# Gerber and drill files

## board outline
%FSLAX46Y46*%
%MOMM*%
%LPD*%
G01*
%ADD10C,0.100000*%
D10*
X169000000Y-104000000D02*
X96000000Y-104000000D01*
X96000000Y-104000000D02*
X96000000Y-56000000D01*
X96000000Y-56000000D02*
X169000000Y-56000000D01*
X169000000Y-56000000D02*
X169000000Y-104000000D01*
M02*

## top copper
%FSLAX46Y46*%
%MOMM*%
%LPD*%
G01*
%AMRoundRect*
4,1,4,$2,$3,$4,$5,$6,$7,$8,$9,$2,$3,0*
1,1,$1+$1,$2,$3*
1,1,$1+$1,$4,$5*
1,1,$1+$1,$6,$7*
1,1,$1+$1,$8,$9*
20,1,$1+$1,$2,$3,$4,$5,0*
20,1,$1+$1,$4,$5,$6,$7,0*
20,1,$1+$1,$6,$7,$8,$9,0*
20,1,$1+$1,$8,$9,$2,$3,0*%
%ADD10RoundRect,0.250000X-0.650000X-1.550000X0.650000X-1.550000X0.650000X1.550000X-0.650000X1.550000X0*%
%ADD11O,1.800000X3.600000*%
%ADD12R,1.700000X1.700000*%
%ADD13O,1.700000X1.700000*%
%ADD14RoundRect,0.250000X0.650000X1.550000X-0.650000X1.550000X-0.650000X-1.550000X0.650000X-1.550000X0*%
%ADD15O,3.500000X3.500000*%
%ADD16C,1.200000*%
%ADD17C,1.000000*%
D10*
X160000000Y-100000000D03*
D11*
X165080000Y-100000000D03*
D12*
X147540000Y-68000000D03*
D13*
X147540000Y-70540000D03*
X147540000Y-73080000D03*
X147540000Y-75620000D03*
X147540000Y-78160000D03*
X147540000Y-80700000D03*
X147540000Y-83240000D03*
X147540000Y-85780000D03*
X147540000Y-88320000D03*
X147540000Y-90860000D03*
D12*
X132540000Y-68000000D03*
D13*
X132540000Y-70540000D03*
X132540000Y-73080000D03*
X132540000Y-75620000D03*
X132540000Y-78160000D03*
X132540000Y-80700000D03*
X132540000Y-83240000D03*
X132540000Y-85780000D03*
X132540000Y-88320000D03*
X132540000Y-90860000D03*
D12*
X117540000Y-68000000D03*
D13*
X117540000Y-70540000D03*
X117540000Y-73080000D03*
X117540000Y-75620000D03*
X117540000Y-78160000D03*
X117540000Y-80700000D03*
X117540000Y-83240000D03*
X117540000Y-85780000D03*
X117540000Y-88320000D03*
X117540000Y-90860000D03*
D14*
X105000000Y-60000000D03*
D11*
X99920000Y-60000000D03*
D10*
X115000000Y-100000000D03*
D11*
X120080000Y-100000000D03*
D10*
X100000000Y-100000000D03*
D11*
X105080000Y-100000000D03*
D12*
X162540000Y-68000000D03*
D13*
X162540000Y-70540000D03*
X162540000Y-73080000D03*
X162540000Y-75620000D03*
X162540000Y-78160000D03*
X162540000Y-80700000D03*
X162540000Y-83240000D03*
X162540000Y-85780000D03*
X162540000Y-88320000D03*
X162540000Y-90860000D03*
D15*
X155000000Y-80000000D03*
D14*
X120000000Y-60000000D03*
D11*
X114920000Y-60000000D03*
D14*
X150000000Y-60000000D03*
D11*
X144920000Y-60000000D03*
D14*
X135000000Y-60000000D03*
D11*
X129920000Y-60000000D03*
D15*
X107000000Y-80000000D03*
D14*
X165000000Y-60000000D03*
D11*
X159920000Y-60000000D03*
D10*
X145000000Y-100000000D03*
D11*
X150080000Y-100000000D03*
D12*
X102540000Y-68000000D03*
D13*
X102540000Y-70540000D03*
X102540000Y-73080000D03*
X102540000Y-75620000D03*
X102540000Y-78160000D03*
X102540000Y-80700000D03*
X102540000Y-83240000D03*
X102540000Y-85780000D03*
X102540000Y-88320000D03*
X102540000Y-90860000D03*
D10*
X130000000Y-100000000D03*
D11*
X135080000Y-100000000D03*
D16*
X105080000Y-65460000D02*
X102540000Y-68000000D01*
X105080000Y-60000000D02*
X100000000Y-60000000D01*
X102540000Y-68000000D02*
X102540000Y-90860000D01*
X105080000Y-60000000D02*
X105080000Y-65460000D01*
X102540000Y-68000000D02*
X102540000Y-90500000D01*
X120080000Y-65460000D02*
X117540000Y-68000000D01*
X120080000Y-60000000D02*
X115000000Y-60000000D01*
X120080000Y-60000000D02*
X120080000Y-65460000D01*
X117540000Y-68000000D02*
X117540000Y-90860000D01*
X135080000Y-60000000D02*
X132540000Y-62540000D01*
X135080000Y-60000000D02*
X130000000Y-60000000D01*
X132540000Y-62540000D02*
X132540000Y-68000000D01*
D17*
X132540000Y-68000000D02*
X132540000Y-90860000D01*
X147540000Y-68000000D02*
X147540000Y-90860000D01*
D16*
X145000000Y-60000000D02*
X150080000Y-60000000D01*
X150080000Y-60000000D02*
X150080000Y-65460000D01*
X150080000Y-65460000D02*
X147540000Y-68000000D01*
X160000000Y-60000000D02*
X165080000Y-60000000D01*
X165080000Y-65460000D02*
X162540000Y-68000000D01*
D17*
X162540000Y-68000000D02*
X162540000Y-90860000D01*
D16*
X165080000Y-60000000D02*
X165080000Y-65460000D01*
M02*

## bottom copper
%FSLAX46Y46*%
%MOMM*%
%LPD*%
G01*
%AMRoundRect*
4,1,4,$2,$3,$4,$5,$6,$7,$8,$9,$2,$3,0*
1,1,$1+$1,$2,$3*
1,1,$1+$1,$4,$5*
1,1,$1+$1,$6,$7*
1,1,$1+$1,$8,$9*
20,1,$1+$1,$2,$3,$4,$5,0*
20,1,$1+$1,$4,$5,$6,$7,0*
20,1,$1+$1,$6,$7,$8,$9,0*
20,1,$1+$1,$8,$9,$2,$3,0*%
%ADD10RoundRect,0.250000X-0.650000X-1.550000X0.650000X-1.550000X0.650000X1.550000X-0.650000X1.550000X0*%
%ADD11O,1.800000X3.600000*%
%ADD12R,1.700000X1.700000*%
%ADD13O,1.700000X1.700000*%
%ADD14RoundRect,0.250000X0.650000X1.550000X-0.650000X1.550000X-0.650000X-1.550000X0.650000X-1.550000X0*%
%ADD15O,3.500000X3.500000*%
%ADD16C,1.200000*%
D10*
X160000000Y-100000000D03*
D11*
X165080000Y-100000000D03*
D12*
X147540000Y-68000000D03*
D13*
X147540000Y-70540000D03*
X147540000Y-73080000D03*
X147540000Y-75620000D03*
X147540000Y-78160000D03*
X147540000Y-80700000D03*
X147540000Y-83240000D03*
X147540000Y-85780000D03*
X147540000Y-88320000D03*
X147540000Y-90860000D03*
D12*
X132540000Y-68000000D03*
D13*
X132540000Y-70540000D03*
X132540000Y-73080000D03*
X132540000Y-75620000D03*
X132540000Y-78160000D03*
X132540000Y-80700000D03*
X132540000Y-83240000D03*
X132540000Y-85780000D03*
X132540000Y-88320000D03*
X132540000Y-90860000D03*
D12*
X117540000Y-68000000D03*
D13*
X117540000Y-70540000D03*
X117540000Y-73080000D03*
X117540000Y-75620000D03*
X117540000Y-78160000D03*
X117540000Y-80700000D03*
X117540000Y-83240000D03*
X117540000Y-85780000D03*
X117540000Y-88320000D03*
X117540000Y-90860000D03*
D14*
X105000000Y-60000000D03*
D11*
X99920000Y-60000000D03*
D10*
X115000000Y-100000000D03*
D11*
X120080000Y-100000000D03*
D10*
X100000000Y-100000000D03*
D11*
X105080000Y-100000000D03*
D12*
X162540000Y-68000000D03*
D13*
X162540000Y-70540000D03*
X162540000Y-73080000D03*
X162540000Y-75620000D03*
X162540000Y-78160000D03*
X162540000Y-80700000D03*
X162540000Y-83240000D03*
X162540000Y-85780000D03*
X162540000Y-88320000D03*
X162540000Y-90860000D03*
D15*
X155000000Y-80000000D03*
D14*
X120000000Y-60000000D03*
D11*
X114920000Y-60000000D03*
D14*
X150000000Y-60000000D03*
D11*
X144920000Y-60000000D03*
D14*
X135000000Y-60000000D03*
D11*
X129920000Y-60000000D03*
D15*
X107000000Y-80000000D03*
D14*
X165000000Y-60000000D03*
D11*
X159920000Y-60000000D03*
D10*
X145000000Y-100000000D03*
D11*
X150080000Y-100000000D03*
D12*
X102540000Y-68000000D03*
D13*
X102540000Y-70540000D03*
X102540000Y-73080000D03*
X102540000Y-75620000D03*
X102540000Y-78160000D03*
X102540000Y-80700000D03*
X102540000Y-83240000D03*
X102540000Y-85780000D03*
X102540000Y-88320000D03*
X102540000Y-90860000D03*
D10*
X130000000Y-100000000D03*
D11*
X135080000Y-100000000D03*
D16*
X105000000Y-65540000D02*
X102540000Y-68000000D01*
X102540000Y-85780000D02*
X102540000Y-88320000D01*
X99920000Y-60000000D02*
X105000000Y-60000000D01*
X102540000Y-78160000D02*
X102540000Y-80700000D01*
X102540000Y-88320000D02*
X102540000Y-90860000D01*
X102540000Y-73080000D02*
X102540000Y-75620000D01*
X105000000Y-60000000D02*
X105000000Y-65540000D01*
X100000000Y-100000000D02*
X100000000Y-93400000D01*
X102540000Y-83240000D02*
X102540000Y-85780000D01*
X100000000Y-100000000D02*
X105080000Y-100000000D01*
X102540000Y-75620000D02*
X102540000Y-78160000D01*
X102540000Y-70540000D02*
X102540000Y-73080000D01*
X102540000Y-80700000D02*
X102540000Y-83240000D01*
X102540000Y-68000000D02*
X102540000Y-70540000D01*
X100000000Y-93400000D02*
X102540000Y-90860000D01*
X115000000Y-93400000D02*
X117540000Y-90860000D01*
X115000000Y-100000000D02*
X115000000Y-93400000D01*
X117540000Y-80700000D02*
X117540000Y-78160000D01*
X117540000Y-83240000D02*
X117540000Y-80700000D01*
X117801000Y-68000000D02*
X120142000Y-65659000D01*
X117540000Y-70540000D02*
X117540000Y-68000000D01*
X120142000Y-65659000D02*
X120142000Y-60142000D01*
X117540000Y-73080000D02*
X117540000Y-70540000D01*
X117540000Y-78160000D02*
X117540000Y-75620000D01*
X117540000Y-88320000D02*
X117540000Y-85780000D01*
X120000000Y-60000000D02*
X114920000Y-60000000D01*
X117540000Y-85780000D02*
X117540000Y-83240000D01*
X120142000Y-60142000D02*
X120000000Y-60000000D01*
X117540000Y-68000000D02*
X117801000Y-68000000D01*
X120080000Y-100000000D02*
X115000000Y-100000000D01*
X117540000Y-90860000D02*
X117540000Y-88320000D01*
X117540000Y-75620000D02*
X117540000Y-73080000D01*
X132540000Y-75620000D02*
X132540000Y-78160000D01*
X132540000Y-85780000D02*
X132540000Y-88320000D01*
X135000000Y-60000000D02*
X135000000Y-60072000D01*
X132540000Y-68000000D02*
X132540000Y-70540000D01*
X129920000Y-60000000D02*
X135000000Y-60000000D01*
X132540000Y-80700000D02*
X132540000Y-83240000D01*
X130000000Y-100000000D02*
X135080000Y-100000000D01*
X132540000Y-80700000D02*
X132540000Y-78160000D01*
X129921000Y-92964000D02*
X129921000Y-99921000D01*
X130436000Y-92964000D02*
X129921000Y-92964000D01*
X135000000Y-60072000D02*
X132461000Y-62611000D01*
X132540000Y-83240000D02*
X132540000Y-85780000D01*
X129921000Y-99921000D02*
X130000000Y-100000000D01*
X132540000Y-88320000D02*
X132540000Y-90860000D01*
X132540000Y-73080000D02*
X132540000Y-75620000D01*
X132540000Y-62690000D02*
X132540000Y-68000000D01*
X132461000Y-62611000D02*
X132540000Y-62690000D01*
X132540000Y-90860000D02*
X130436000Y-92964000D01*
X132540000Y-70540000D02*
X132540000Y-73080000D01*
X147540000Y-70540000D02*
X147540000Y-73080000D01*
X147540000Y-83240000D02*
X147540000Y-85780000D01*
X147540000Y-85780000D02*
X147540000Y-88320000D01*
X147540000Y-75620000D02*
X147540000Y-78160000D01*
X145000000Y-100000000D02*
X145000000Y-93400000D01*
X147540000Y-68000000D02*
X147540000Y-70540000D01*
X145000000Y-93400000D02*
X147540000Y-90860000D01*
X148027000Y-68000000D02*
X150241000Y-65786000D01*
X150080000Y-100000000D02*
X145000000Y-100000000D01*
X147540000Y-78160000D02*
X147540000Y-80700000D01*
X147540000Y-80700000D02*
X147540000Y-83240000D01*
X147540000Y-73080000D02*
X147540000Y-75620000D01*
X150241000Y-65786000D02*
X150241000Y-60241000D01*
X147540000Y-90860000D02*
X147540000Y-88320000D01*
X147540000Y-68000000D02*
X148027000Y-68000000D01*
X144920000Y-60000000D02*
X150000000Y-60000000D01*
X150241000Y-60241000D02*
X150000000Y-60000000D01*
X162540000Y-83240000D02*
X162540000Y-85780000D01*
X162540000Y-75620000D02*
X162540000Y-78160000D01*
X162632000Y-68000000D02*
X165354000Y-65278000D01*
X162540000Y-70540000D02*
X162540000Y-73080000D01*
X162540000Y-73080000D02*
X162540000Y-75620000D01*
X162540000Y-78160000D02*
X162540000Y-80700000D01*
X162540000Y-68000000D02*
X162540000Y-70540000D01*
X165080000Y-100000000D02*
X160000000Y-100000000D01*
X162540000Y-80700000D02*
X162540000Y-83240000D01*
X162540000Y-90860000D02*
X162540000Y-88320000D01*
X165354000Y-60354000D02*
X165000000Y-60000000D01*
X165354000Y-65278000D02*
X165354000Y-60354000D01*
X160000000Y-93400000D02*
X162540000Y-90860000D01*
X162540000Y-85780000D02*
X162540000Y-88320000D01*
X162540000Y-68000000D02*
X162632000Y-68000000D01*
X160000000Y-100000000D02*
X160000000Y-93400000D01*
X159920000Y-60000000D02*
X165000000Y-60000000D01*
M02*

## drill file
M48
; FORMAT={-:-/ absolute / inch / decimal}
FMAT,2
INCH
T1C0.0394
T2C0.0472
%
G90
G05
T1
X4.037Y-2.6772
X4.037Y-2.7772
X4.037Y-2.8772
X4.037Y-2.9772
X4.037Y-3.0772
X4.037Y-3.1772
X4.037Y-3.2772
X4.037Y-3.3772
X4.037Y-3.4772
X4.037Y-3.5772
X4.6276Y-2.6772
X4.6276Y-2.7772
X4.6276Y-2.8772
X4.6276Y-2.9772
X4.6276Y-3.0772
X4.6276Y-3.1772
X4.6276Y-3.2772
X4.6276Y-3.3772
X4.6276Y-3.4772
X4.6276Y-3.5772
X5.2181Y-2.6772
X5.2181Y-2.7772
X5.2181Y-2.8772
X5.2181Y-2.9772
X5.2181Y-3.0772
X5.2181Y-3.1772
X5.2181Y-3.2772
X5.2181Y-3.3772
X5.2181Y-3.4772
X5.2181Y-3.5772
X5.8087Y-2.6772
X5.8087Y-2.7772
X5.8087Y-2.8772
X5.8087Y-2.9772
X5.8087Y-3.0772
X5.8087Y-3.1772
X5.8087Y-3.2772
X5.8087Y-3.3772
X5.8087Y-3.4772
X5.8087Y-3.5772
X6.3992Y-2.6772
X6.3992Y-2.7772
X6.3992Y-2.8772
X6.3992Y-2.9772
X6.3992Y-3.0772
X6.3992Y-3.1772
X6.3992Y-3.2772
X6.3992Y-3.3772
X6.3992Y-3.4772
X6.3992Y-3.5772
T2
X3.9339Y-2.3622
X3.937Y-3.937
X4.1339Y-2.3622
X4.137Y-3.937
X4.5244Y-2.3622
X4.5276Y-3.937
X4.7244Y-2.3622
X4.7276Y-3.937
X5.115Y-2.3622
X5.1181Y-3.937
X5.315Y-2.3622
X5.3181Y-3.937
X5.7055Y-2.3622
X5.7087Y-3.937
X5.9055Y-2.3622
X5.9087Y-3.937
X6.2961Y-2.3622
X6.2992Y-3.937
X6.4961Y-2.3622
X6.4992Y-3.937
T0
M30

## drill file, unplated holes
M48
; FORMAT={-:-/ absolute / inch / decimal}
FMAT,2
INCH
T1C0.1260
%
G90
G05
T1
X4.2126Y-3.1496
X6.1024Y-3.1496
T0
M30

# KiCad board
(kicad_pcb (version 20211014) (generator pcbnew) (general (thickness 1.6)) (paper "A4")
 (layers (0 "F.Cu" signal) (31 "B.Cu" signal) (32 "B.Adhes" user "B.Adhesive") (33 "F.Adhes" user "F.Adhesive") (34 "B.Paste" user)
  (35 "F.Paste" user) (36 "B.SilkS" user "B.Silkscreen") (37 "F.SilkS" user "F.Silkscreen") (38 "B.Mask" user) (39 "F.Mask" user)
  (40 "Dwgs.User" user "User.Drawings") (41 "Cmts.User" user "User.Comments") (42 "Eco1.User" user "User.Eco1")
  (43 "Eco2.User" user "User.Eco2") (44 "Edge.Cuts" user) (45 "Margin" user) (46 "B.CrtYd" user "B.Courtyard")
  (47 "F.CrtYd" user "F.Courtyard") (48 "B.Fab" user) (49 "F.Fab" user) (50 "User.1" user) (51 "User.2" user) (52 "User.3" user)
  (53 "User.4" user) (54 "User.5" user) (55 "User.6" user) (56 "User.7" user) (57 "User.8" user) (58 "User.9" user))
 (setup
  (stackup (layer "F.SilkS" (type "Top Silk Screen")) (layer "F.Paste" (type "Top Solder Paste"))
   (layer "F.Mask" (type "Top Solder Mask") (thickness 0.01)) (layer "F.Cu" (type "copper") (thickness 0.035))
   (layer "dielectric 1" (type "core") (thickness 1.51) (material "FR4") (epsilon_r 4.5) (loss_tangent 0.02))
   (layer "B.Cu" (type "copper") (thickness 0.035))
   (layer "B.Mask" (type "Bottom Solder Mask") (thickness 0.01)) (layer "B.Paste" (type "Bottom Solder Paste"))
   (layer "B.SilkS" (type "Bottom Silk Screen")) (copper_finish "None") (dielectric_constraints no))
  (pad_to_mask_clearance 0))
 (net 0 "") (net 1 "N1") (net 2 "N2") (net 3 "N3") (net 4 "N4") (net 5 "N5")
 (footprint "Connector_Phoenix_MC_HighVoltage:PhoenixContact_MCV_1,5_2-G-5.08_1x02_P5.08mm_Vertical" (layer "F.Cu") (at 160 100)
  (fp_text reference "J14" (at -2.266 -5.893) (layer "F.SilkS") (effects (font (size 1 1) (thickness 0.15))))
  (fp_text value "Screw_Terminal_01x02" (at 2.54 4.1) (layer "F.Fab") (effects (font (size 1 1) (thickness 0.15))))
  (pad "1" thru_hole roundrect (at 0 0) (size 1.8 3.6) (drill 1.2) (layers *.Cu *.Mask) (roundrect_rratio 0.1388888889) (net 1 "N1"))
  (pad "2" thru_hole oval (at 5.08 0) (size 1.8 3.6) (drill 1.2) (layers *.Cu *.Mask) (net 1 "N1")))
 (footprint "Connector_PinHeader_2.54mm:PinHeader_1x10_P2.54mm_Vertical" (layer "F.Cu") (at 147.54 68)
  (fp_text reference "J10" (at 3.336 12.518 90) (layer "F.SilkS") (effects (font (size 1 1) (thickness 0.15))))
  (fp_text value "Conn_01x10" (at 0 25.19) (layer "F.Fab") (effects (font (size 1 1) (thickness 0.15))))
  (pad "1" thru_hole rect (at 0 0) (size 1.7 1.7) (drill 1) (layers *.Cu *.Mask) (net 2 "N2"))
  (pad "2" thru_hole oval (at 0 2.54) (size 1.7 1.7) (drill 1) (layers *.Cu *.Mask) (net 2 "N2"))
  (pad "3" thru_hole oval (at 0 5.08) (size 1.7 1.7) (drill 1) (layers *.Cu *.Mask) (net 2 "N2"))
  (pad "4" thru_hole oval (at 0 7.62) (size 1.7 1.7) (drill 1) (layers *.Cu *.Mask) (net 2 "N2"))
  (pad "5" thru_hole oval (at 0 10.16) (size 1.7 1.7) (drill 1) (layers *.Cu *.Mask) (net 2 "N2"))
  (pad "6" thru_hole oval (at 0 12.7) (size 1.7 1.7) (drill 1) (layers *.Cu *.Mask) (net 2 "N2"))
  (pad "7" thru_hole oval (at 0 15.24) (size 1.7 1.7) (drill 1) (layers *.Cu *.Mask) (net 2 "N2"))
  (pad "8" thru_hole oval (at 0 17.78) (size 1.7 1.7) (drill 1) (layers *.Cu *.Mask) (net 2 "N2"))
  (pad "9" thru_hole oval (at 0 20.32) (size 1.7 1.7) (drill 1) (layers *.Cu *.Mask) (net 2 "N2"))
  (pad "10" thru_hole oval (at 0 22.86) (size 1.7 1.7) (drill 1) (layers *.Cu *.Mask) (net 2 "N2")))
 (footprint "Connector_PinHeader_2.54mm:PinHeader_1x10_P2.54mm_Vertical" (layer "F.Cu") (at 132.54 68)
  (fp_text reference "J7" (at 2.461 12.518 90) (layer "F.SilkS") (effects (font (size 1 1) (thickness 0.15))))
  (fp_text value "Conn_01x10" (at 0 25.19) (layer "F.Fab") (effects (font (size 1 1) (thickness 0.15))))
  (pad "1" thru_hole rect (at 0 0) (size 1.7 1.7) (drill 1) (layers *.Cu *.Mask) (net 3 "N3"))
  (pad "2" thru_hole oval (at 0 2.54) (size 1.7 1.7) (drill 1) (layers *.Cu *.Mask) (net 3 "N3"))
  (pad "3" thru_hole oval (at 0 5.08) (size 1.7 1.7) (drill 1) (layers *.Cu *.Mask) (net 3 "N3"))
  (pad "4" thru_hole oval (at 0 7.62) (size 1.7 1.7) (drill 1) (layers *.Cu *.Mask) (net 3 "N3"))
  (pad "5" thru_hole oval (at 0 10.16) (size 1.7 1.7) (drill 1) (layers *.Cu *.Mask) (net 3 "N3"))
  (pad "6" thru_hole oval (at 0 12.7) (size 1.7 1.7) (drill 1) (layers *.Cu *.Mask) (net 3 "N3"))
  (pad "7" thru_hole oval (at 0 15.24) (size 1.7 1.7) (drill 1) (layers *.Cu *.Mask) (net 3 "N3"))
  (pad "8" thru_hole oval (at 0 17.78) (size 1.7 1.7) (drill 1) (layers *.Cu *.Mask) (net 3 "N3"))
  (pad "9" thru_hole oval (at 0 20.32) (size 1.7 1.7) (drill 1) (layers *.Cu *.Mask) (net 3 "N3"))
  (pad "10" thru_hole oval (at 0 22.86) (size 1.7 1.7) (drill 1) (layers *.Cu *.Mask) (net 3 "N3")))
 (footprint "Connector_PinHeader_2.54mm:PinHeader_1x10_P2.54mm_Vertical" (layer "F.Cu") (at 117.54 68)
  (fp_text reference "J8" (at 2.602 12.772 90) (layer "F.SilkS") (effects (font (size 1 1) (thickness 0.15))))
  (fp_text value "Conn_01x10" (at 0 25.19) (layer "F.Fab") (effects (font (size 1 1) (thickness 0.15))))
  (pad "1" thru_hole rect (at 0 0) (size 1.7 1.7) (drill 1) (layers *.Cu *.Mask) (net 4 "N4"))
  (pad "2" thru_hole oval (at 0 2.54) (size 1.7 1.7) (drill 1) (layers *.Cu *.Mask) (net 4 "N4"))
  (pad "3" thru_hole oval (at 0 5.08) (size 1.7 1.7) (drill 1) (layers *.Cu *.Mask) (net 4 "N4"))
  (pad "4" thru_hole oval (at 0 7.62) (size 1.7 1.7) (drill 1) (layers *.Cu *.Mask) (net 4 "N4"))
  (pad "5" thru_hole oval (at 0 10.16) (size 1.7 1.7) (drill 1) (layers *.Cu *.Mask) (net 4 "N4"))
  (pad "6" thru_hole oval (at 0 12.7) (size 1.7 1.7) (drill 1) (layers *.Cu *.Mask) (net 4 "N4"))
  (pad "7" thru_hole oval (at 0 15.24) (size 1.7 1.7) (drill 1) (layers *.Cu *.Mask) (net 4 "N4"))
  (pad "8" thru_hole oval (at 0 17.78) (size 1.7 1.7) (drill 1) (layers *.Cu *.Mask) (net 4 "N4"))
  (pad "9" thru_hole oval (at 0 20.32) (size 1.7 1.7) (drill 1) (layers *.Cu *.Mask) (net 4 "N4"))
  (pad "10" thru_hole oval (at 0 22.86) (size 1.7 1.7) (drill 1) (layers *.Cu *.Mask) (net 4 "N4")))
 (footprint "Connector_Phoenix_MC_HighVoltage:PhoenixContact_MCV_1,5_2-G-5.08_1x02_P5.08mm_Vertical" (layer "F.Cu") (at 105 60 180)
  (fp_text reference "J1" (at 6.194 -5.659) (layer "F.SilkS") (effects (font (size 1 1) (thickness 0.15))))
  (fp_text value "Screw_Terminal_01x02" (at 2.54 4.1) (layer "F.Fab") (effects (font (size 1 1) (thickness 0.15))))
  (pad "1" thru_hole roundrect (at 0 0 180) (size 1.8 3.6) (drill 1.2) (layers *.Cu *.Mask) (roundrect_rratio 0.1388888889) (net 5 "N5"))
  (pad "2" thru_hole oval (at 5.08 0 180) (size 1.8 3.6) (drill 1.2) (layers *.Cu *.Mask) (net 5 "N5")))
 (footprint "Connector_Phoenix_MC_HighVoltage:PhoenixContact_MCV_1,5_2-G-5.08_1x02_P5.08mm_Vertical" (layer "F.Cu") (at 115 100)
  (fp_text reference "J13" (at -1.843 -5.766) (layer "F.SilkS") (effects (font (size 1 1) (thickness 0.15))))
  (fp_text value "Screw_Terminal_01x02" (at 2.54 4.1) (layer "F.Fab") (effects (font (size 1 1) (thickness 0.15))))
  (pad "1" thru_hole roundrect (at 0 0) (size 1.8 3.6) (drill 1.2) (layers *.Cu *.Mask) (roundrect_rratio 0.1388888889) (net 4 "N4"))
  (pad "2" thru_hole oval (at 5.08 0) (size 1.8 3.6) (drill 1.2) (layers *.Cu *.Mask) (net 4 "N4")))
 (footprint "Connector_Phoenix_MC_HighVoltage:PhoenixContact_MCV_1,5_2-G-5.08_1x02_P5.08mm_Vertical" (layer "F.Cu") (at 100 100)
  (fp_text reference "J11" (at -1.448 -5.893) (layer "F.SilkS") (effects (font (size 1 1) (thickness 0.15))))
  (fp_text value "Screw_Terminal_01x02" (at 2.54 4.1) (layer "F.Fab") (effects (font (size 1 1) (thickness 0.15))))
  (pad "1" thru_hole roundrect (at 0 0) (size 1.8 3.6) (drill 1.2) (layers *.Cu *.Mask) (roundrect_rratio 0.1388888889) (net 5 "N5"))
  (pad "2" thru_hole oval (at 5.08 0) (size 1.8 3.6) (drill 1.2) (layers *.Cu *.Mask) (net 5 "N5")))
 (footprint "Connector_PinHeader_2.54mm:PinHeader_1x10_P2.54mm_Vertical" (layer "F.Cu") (at 162.54 68)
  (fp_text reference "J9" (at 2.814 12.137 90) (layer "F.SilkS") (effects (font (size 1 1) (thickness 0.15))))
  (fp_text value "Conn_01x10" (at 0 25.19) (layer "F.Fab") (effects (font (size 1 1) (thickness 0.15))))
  (pad "1" thru_hole rect (at 0 0) (size 1.7 1.7) (drill 1) (layers *.Cu *.Mask) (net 1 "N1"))
  (pad "2" thru_hole oval (at 0 2.54) (size 1.7 1.7) (drill 1) (layers *.Cu *.Mask) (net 1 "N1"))
  (pad "3" thru_hole oval (at 0 5.08) (size 1.7 1.7) (drill 1) (layers *.Cu *.Mask) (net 1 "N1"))
  (pad "4" thru_hole oval (at 0 7.62) (size 1.7 1.7) (drill 1) (layers *.Cu *.Mask) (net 1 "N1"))
  (pad "5" thru_hole oval (at 0 10.16) (size 1.7 1.7) (drill 1) (layers *.Cu *.Mask) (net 1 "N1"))
  (pad "6" thru_hole oval (at 0 12.7) (size 1.7 1.7) (drill 1) (layers *.Cu *.Mask) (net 1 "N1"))
  (pad "7" thru_hole oval (at 0 15.24) (size 1.7 1.7) (drill 1) (layers *.Cu *.Mask) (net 1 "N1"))
  (pad "8" thru_hole oval (at 0 17.78) (size 1.7 1.7) (drill 1) (layers *.Cu *.Mask) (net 1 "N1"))
  (pad "9" thru_hole oval (at 0 20.32) (size 1.7 1.7) (drill 1) (layers *.Cu *.Mask) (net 1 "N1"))
  (pad "10" thru_hole oval (at 0 22.86) (size 1.7 1.7) (drill 1) (layers *.Cu *.Mask) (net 1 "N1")))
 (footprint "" (layer "F.Cu") (at 154.178 80.137)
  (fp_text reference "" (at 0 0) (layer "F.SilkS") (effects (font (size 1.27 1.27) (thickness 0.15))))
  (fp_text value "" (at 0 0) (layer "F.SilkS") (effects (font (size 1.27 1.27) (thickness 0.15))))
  (pad "" np_thru_hole oval (at 0.822 -0.137) (size 3.5 3.5) (drill 3.2) (layers F&B.Cu *.Mask)))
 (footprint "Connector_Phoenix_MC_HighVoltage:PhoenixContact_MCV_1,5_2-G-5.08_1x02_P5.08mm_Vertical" (layer "F.Cu") (at 120 60 180)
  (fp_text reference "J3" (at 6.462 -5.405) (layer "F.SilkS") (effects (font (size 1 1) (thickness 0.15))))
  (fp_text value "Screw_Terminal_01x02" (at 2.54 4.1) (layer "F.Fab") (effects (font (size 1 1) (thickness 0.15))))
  (pad "1" thru_hole roundrect (at 0 0 180) (size 1.8 3.6) (drill 1.2) (layers *.Cu *.Mask) (roundrect_rratio 0.1388888889) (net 4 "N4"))
  (pad "2" thru_hole oval (at 5.08 0 180) (size 1.8 3.6) (drill 1.2) (layers *.Cu *.Mask) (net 4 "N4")))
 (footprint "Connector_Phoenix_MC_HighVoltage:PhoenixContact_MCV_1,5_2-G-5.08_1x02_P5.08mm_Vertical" (layer "F.Cu") (at 150 60 180)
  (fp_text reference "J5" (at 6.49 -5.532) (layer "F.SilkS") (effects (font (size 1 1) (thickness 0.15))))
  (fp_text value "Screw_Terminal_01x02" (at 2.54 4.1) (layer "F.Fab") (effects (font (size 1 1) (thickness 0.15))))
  (pad "1" thru_hole roundrect (at 0 0 180) (size 1.8 3.6) (drill 1.2) (layers *.Cu *.Mask) (roundrect_rratio 0.1388888889) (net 2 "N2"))
  (pad "2" thru_hole oval (at 5.08 0 180) (size 1.8 3.6) (drill 1.2) (layers *.Cu *.Mask) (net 2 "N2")))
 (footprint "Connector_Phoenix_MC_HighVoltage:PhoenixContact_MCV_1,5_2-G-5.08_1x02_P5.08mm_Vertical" (layer "F.Cu") (at 135 60 180)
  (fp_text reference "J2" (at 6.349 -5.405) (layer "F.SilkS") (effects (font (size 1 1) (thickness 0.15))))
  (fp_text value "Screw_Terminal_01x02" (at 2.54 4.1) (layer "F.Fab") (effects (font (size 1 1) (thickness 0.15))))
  (pad "1" thru_hole roundrect (at 0 0 180) (size 1.8 3.6) (drill 1.2) (layers *.Cu *.Mask) (roundrect_rratio 0.1388888889) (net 3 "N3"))
  (pad "2" thru_hole oval (at 5.08 0 180) (size 1.8 3.6) (drill 1.2) (layers *.Cu *.Mask) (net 3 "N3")))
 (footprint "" (layer "F.Cu") (at 107.823 80.264)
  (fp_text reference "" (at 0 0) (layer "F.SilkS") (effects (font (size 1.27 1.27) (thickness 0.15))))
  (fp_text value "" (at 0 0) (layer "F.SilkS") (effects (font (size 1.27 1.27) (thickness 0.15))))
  (pad "" np_thru_hole oval (at -0.823 -0.264) (size 3.5 3.5) (drill 3.2) (layers F&B.Cu *.Mask)))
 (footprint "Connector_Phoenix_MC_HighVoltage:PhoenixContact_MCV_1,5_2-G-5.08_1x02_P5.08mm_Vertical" (layer "F.Cu") (at 165 60 180)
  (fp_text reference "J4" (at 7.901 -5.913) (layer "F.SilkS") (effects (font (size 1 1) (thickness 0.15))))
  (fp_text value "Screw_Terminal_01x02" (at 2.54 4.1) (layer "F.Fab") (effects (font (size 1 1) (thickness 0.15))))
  (pad "1" thru_hole roundrect (at 0 0 180) (size 1.8 3.6) (drill 1.2) (layers *.Cu *.Mask) (roundrect_rratio 0.1388888889) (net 1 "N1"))
  (pad "2" thru_hole oval (at 5.08 0 180) (size 1.8 3.6) (drill 1.2) (layers *.Cu *.Mask) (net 1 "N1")))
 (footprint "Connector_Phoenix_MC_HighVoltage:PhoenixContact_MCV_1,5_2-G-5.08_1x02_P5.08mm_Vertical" (layer "F.Cu") (at 145 100)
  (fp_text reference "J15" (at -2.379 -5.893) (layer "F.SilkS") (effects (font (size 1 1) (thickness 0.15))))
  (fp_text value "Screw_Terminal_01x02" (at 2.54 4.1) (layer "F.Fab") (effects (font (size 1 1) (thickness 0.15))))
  (pad "1" thru_hole roundrect (at 0 0) (size 1.8 3.6) (drill 1.2) (layers *.Cu *.Mask) (roundrect_rratio 0.1388888889) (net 2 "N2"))
  (pad "2" thru_hole oval (at 5.08 0) (size 1.8 3.6) (drill 1.2) (layers *.Cu *.Mask) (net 2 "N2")))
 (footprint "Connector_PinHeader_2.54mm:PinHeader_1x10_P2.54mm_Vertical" (layer "F.Cu") (at 102.54 68)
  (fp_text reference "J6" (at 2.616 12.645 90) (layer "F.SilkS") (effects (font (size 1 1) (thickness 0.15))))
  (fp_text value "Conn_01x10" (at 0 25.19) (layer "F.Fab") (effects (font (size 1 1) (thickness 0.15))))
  (pad "1" thru_hole rect (at 0 0) (size 1.7 1.7) (drill 1) (layers *.Cu *.Mask) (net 5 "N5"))
  (pad "2" thru_hole oval (at 0 2.54) (size 1.7 1.7) (drill 1) (layers *.Cu *.Mask) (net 5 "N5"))
  (pad "3" thru_hole oval (at 0 5.08) (size 1.7 1.7) (drill 1) (layers *.Cu *.Mask) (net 5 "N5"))
  (pad "4" thru_hole oval (at 0 7.62) (size 1.7 1.7) (drill 1) (layers *.Cu *.Mask) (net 5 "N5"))
  (pad "5" thru_hole oval (at 0 10.16) (size 1.7 1.7) (drill 1) (layers *.Cu *.Mask) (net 5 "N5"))
  (pad "6" thru_hole oval (at 0 12.7) (size 1.7 1.7) (drill 1) (layers *.Cu *.Mask) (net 5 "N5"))
  (pad "7" thru_hole oval (at 0 15.24) (size 1.7 1.7) (drill 1) (layers *.Cu *.Mask) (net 5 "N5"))
  (pad "8" thru_hole oval (at 0 17.78) (size 1.7 1.7) (drill 1) (layers *.Cu *.Mask) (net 5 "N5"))
  (pad "9" thru_hole oval (at 0 20.32) (size 1.7 1.7) (drill 1) (layers *.Cu *.Mask) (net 5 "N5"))
  (pad "10" thru_hole oval (at 0 22.86) (size 1.7 1.7) (drill 1) (layers *.Cu *.Mask) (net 5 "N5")))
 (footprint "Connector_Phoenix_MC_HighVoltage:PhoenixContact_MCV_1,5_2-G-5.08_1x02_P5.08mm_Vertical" (layer "F.Cu") (at 130 100)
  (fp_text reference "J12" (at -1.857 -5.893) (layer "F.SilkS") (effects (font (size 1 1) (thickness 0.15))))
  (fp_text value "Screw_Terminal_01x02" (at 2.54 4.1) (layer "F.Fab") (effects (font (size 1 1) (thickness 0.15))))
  (pad "1" thru_hole roundrect (at 0 0) (size 1.8 3.6) (drill 1.2) (layers *.Cu *.Mask) (roundrect_rratio 0.1388888889) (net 3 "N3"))
  (pad "2" thru_hole oval (at 5.08 0) (size 1.8 3.6) (drill 1.2) (layers *.Cu *.Mask) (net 3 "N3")))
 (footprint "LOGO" (layer "B.Cu") (at 125.095 80.264 -90)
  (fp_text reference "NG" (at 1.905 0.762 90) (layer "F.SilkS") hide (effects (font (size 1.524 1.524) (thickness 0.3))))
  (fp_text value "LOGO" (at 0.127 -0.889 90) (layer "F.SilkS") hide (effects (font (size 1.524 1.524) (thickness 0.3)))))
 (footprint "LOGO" (layer "B.Cu") (at 138.176 80.391 90)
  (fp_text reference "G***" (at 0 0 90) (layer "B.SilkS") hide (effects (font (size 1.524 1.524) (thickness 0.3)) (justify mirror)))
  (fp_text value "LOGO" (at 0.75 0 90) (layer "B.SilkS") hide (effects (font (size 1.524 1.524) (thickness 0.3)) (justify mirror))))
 (gr_rect (start 169 104) (end 96 56) (layer "Edge.Cuts") (width 0.1) (fill none))
 (segment (start 105.08 65.46) (end 102.54 68) (width 1.2) (layer "F.Cu") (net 5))
 (segment (start 105.08 60) (end 100 60) (width 1.2) (layer "F.Cu") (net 5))
 (segment (start 102.54 68) (end 102.54 90.86) (width 1.2) (layer "F.Cu") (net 5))
 (segment (start 105.08 60) (end 105.08 65.46) (width 1.2) (layer "F.Cu") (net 5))
 (segment (start 102.54 68) (end 102.54 90.5) (width 1.2) (layer "F.Cu") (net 5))
 (segment (start 105 65.54) (end 102.54 68) (width 1.2) (layer "B.Cu") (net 5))
 (segment (start 102.54 85.78) (end 102.54 88.32) (width 1.2) (layer "B.Cu") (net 5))
 (segment (start 99.92 60) (end 105 60) (width 1.2) (layer "B.Cu") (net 5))
 (segment (start 102.54 78.16) (end 102.54 80.7) (width 1.2) (layer "B.Cu") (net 5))
 (segment (start 102.54 88.32) (end 102.54 90.86) (width 1.2) (layer "B.Cu") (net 5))
 (segment (start 102.54 73.08) (end 102.54 75.62) (width 1.2) (layer "B.Cu") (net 5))
 (segment (start 105 60) (end 105 65.54) (width 1.2) (layer "B.Cu") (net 5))
 (segment (start 100 100) (end 100 93.4) (width 1.2) (layer "B.Cu") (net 5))
 (segment (start 102.54 83.24) (end 102.54 85.78) (width 1.2) (layer "B.Cu") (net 5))
 (segment (start 100 100) (end 105.08 100) (width 1.2) (layer "B.Cu") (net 5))
 (segment (start 102.54 75.62) (end 102.54 78.16) (width 1.2) (layer "B.Cu") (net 5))
 (segment (start 102.54 70.54) (end 102.54 73.08) (width 1.2) (layer "B.Cu") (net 5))
 (segment (start 102.54 80.7) (end 102.54 83.24) (width 1.2) (layer "B.Cu") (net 5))
 (segment (start 102.54 68) (end 102.54 70.54) (width 1.2) (layer "B.Cu") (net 5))
 (segment (start 100 93.4) (end 102.54 90.86) (width 1.2) (layer "B.Cu") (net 5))
 (segment (start 120.08 65.46) (end 117.54 68) (width 1.2) (layer "F.Cu") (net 4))
 (segment (start 120.08 60) (end 115 60) (width 1.2) (layer "F.Cu") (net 4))
 (segment (start 120.08 60) (end 120.08 65.46) (width 1.2) (layer "F.Cu") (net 4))
 (segment (start 117.54 68) (end 117.54 90.86) (width 1.2) (layer "F.Cu") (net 4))
 (segment (start 115 93.4) (end 117.54 90.86) (width 1.2) (layer "B.Cu") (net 4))
 (segment (start 115 100) (end 115 93.4) (width 1.2) (layer "B.Cu") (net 4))
 (segment (start 117.54 80.7) (end 117.54 78.16) (width 1.2) (layer "B.Cu") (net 4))
 (segment (start 117.54 83.24) (end 117.54 80.7) (width 1.2) (layer "B.Cu") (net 4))
 (segment (start 117.801 68) (end 120.142 65.659) (width 1.2) (layer "B.Cu") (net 4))
 (segment (start 117.54 70.54) (end 117.54 68) (width 1.2) (layer "B.Cu") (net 4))
 (segment (start 120.142 65.659) (end 120.142 60.142) (width 1.2) (layer "B.Cu") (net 4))
 (segment (start 117.54 73.08) (end 117.54 70.54) (width 1.2) (layer "B.Cu") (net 4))
 (segment (start 117.54 78.16) (end 117.54 75.62) (width 1.2) (layer "B.Cu") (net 4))
 (segment (start 117.54 88.32) (end 117.54 85.78) (width 1.2) (layer "B.Cu") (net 4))
 (segment (start 120 60) (end 114.92 60) (width 1.2) (layer "B.Cu") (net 4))
 (segment (start 117.54 85.78) (end 117.54 83.24) (width 1.2) (layer "B.Cu") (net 4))
 (segment (start 120.142 60.142) (end 120 60) (width 1.2) (layer "B.Cu") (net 4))
 (segment (start 117.54 68) (end 117.801 68) (width 1.2) (layer "B.Cu") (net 4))
 (segment (start 120.08 100) (end 115 100) (width 1.2) (layer "B.Cu") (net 4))
 (segment (start 117.54 90.86) (end 117.54 88.32) (width 1.2) (layer "B.Cu") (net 4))
 (segment (start 117.54 75.62) (end 117.54 73.08) (width 1.2) (layer "B.Cu") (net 4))
 (segment (start 135.08 60) (end 132.54 62.54) (width 1.2) (layer "F.Cu") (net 3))
 (segment (start 135.08 60) (end 130 60) (width 1.2) (layer "F.Cu") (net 3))
 (segment (start 132.54 62.54) (end 132.54 68) (width 1.2) (layer "F.Cu") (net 3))
 (segment (start 132.54 68) (end 132.54 90.86) (width 1) (layer "F.Cu") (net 3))
 (segment (start 132.54 75.62) (end 132.54 78.16) (width 1.2) (layer "B.Cu") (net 3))
 (segment (start 132.54 85.78) (end 132.54 88.32) (width 1.2) (layer "B.Cu") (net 3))
 (segment (start 135 60) (end 135 60.072) (width 1.2) (layer "B.Cu") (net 3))
 (segment (start 132.54 68) (end 132.54 70.54) (width 1.2) (layer "B.Cu") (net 3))
 (segment (start 129.92 60) (end 135 60) (width 1.2) (layer "B.Cu") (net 3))
 (segment (start 132.54 80.7) (end 132.54 83.24) (width 1.2) (layer "B.Cu") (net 3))
 (segment (start 130 100) (end 135.08 100) (width 1.2) (layer "B.Cu") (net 3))
 (segment (start 132.54 80.7) (end 132.54 78.16) (width 1.2) (layer "B.Cu") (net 3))
 (segment (start 129.921 92.964) (end 129.921 99.921) (width 1.2) (layer "B.Cu") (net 3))
 (segment (start 130.436 92.964) (end 129.921 92.964) (width 1.2) (layer "B.Cu") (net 3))
 (segment (start 135 60.072) (end 132.461 62.611) (width 1.2) (layer "B.Cu") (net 3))
 (segment (start 132.54 83.24) (end 132.54 85.78) (width 1.2) (layer "B.Cu") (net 3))
 (segment (start 129.921 99.921) (end 130 100) (width 1.2) (layer "B.Cu") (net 3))
 (segment (start 132.54 88.32) (end 132.54 90.86) (width 1.2) (layer "B.Cu") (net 3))
 (segment (start 132.54 73.08) (end 132.54 75.62) (width 1.2) (layer "B.Cu") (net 3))
 (segment (start 132.54 62.69) (end 132.54 68) (width 1.2) (layer "B.Cu") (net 3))
 (segment (start 132.461 62.611) (end 132.54 62.69) (width 1.2) (layer "B.Cu") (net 3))
 (segment (start 132.54 90.86) (end 130.436 92.964) (width 1.2) (layer "B.Cu") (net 3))
 (segment (start 132.54 70.54) (end 132.54 73.08) (width 1.2) (layer "B.Cu") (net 3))
 (segment (start 147.54 68) (end 147.54 90.86) (width 1) (layer "F.Cu") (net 2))
 (segment (start 145 60) (end 150.08 60) (width 1.2) (layer "F.Cu") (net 2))
 (segment (start 150.08 60) (end 150.08 65.46) (width 1.2) (layer "F.Cu") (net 2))
 (segment (start 150.08 65.46) (end 147.54 68) (width 1.2) (layer "F.Cu") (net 2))
 (segment (start 147.54 70.54) (end 147.54 73.08) (width 1.2) (layer "B.Cu") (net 2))
 (segment (start 147.54 83.24) (end 147.54 85.78) (width 1.2) (layer "B.Cu") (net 2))
 (segment (start 147.54 85.78) (end 147.54 88.32) (width 1.2) (layer "B.Cu") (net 2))
 (segment (start 147.54 75.62) (end 147.54 78.16) (width 1.2) (layer "B.Cu") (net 2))
 (segment (start 145 100) (end 145 93.4) (width 1.2) (layer "B.Cu") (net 2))
 (segment (start 147.54 68) (end 147.54 70.54) (width 1.2) (layer "B.Cu") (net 2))
 (segment (start 145 93.4) (end 147.54 90.86) (width 1.2) (layer "B.Cu") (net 2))
 (segment (start 148.027 68) (end 150.241 65.786) (width 1.2) (layer "B.Cu") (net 2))
 (segment (start 150.08 100) (end 145 100) (width 1.2) (layer "B.Cu") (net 2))
 (segment (start 147.54 78.16) (end 147.54 80.7) (width 1.2) (layer "B.Cu") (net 2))
 (segment (start 147.54 80.7) (end 147.54 83.24) (width 1.2) (layer "B.Cu") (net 2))
 (segment (start 147.54 73.08) (end 147.54 75.62) (width 1.2) (layer "B.Cu") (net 2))
 (segment (start 150.241 65.786) (end 150.241 60.241) (width 1.2) (layer "B.Cu") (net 2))
 (segment (start 147.54 90.86) (end 147.54 88.32) (width 1.2) (layer "B.Cu") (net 2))
 (segment (start 147.54 68) (end 148.027 68) (width 1.2) (layer "B.Cu") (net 2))
 (segment (start 144.92 60) (end 150 60) (width 1.2) (layer "B.Cu") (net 2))
 (segment (start 150.241 60.241) (end 150 60) (width 1.2) (layer "B.Cu") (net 2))
 (segment (start 160 60) (end 165.08 60) (width 1.2) (layer "F.Cu") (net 1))
 (segment (start 165.08 65.46) (end 162.54 68) (width 1.2) (layer "F.Cu") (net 1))
 (segment (start 162.54 68) (end 162.54 90.86) (width 1) (layer "F.Cu") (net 1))
 (segment (start 165.08 60) (end 165.08 65.46) (width 1.2) (layer "F.Cu") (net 1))
 (segment (start 162.54 83.24) (end 162.54 85.78) (width 1.2) (layer "B.Cu") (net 1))
 (segment (start 162.54 75.62) (end 162.54 78.16) (width 1.2) (layer "B.Cu") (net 1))
 (segment (start 162.632 68) (end 165.354 65.278) (width 1.2) (layer "B.Cu") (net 1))
 (segment (start 162.54 70.54) (end 162.54 73.08) (width 1.2) (layer "B.Cu") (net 1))
 (segment (start 162.54 73.08) (end 162.54 75.62) (width 1.2) (layer "B.Cu") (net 1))
 (segment (start 162.54 78.16) (end 162.54 80.7) (width 1.2) (layer "B.Cu") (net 1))
 (segment (start 162.54 68) (end 162.54 70.54) (width 1.2) (layer "B.Cu") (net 1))
 (segment (start 165.08 100) (end 160 100) (width 1.2) (layer "B.Cu") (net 1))
 (segment (start 162.54 80.7) (end 162.54 83.24) (width 1.2) (layer "B.Cu") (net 1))
 (segment (start 162.54 90.86) (end 162.54 88.32) (width 1.2) (layer "B.Cu") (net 1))
 (segment (start 165.354 60.354) (end 165 60) (width 1.2) (layer "B.Cu") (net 1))
 (segment (start 165.354 65.278) (end 165.354 60.354) (width 1.2) (layer "B.Cu") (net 1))
 (segment (start 160 93.4) (end 162.54 90.86) (width 1.2) (layer "B.Cu") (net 1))
 (segment (start 162.54 85.78) (end 162.54 88.32) (width 1.2) (layer "B.Cu") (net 1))
 (segment (start 162.54 68) (end 162.632 68) (width 1.2) (layer "B.Cu") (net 1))
 (segment (start 160 100) (end 160 93.4) (width 1.2) (layer "B.Cu") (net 1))
 (segment (start 159.92 60) (end 165 60) (width 1.2) (layer "B.Cu") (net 1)))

